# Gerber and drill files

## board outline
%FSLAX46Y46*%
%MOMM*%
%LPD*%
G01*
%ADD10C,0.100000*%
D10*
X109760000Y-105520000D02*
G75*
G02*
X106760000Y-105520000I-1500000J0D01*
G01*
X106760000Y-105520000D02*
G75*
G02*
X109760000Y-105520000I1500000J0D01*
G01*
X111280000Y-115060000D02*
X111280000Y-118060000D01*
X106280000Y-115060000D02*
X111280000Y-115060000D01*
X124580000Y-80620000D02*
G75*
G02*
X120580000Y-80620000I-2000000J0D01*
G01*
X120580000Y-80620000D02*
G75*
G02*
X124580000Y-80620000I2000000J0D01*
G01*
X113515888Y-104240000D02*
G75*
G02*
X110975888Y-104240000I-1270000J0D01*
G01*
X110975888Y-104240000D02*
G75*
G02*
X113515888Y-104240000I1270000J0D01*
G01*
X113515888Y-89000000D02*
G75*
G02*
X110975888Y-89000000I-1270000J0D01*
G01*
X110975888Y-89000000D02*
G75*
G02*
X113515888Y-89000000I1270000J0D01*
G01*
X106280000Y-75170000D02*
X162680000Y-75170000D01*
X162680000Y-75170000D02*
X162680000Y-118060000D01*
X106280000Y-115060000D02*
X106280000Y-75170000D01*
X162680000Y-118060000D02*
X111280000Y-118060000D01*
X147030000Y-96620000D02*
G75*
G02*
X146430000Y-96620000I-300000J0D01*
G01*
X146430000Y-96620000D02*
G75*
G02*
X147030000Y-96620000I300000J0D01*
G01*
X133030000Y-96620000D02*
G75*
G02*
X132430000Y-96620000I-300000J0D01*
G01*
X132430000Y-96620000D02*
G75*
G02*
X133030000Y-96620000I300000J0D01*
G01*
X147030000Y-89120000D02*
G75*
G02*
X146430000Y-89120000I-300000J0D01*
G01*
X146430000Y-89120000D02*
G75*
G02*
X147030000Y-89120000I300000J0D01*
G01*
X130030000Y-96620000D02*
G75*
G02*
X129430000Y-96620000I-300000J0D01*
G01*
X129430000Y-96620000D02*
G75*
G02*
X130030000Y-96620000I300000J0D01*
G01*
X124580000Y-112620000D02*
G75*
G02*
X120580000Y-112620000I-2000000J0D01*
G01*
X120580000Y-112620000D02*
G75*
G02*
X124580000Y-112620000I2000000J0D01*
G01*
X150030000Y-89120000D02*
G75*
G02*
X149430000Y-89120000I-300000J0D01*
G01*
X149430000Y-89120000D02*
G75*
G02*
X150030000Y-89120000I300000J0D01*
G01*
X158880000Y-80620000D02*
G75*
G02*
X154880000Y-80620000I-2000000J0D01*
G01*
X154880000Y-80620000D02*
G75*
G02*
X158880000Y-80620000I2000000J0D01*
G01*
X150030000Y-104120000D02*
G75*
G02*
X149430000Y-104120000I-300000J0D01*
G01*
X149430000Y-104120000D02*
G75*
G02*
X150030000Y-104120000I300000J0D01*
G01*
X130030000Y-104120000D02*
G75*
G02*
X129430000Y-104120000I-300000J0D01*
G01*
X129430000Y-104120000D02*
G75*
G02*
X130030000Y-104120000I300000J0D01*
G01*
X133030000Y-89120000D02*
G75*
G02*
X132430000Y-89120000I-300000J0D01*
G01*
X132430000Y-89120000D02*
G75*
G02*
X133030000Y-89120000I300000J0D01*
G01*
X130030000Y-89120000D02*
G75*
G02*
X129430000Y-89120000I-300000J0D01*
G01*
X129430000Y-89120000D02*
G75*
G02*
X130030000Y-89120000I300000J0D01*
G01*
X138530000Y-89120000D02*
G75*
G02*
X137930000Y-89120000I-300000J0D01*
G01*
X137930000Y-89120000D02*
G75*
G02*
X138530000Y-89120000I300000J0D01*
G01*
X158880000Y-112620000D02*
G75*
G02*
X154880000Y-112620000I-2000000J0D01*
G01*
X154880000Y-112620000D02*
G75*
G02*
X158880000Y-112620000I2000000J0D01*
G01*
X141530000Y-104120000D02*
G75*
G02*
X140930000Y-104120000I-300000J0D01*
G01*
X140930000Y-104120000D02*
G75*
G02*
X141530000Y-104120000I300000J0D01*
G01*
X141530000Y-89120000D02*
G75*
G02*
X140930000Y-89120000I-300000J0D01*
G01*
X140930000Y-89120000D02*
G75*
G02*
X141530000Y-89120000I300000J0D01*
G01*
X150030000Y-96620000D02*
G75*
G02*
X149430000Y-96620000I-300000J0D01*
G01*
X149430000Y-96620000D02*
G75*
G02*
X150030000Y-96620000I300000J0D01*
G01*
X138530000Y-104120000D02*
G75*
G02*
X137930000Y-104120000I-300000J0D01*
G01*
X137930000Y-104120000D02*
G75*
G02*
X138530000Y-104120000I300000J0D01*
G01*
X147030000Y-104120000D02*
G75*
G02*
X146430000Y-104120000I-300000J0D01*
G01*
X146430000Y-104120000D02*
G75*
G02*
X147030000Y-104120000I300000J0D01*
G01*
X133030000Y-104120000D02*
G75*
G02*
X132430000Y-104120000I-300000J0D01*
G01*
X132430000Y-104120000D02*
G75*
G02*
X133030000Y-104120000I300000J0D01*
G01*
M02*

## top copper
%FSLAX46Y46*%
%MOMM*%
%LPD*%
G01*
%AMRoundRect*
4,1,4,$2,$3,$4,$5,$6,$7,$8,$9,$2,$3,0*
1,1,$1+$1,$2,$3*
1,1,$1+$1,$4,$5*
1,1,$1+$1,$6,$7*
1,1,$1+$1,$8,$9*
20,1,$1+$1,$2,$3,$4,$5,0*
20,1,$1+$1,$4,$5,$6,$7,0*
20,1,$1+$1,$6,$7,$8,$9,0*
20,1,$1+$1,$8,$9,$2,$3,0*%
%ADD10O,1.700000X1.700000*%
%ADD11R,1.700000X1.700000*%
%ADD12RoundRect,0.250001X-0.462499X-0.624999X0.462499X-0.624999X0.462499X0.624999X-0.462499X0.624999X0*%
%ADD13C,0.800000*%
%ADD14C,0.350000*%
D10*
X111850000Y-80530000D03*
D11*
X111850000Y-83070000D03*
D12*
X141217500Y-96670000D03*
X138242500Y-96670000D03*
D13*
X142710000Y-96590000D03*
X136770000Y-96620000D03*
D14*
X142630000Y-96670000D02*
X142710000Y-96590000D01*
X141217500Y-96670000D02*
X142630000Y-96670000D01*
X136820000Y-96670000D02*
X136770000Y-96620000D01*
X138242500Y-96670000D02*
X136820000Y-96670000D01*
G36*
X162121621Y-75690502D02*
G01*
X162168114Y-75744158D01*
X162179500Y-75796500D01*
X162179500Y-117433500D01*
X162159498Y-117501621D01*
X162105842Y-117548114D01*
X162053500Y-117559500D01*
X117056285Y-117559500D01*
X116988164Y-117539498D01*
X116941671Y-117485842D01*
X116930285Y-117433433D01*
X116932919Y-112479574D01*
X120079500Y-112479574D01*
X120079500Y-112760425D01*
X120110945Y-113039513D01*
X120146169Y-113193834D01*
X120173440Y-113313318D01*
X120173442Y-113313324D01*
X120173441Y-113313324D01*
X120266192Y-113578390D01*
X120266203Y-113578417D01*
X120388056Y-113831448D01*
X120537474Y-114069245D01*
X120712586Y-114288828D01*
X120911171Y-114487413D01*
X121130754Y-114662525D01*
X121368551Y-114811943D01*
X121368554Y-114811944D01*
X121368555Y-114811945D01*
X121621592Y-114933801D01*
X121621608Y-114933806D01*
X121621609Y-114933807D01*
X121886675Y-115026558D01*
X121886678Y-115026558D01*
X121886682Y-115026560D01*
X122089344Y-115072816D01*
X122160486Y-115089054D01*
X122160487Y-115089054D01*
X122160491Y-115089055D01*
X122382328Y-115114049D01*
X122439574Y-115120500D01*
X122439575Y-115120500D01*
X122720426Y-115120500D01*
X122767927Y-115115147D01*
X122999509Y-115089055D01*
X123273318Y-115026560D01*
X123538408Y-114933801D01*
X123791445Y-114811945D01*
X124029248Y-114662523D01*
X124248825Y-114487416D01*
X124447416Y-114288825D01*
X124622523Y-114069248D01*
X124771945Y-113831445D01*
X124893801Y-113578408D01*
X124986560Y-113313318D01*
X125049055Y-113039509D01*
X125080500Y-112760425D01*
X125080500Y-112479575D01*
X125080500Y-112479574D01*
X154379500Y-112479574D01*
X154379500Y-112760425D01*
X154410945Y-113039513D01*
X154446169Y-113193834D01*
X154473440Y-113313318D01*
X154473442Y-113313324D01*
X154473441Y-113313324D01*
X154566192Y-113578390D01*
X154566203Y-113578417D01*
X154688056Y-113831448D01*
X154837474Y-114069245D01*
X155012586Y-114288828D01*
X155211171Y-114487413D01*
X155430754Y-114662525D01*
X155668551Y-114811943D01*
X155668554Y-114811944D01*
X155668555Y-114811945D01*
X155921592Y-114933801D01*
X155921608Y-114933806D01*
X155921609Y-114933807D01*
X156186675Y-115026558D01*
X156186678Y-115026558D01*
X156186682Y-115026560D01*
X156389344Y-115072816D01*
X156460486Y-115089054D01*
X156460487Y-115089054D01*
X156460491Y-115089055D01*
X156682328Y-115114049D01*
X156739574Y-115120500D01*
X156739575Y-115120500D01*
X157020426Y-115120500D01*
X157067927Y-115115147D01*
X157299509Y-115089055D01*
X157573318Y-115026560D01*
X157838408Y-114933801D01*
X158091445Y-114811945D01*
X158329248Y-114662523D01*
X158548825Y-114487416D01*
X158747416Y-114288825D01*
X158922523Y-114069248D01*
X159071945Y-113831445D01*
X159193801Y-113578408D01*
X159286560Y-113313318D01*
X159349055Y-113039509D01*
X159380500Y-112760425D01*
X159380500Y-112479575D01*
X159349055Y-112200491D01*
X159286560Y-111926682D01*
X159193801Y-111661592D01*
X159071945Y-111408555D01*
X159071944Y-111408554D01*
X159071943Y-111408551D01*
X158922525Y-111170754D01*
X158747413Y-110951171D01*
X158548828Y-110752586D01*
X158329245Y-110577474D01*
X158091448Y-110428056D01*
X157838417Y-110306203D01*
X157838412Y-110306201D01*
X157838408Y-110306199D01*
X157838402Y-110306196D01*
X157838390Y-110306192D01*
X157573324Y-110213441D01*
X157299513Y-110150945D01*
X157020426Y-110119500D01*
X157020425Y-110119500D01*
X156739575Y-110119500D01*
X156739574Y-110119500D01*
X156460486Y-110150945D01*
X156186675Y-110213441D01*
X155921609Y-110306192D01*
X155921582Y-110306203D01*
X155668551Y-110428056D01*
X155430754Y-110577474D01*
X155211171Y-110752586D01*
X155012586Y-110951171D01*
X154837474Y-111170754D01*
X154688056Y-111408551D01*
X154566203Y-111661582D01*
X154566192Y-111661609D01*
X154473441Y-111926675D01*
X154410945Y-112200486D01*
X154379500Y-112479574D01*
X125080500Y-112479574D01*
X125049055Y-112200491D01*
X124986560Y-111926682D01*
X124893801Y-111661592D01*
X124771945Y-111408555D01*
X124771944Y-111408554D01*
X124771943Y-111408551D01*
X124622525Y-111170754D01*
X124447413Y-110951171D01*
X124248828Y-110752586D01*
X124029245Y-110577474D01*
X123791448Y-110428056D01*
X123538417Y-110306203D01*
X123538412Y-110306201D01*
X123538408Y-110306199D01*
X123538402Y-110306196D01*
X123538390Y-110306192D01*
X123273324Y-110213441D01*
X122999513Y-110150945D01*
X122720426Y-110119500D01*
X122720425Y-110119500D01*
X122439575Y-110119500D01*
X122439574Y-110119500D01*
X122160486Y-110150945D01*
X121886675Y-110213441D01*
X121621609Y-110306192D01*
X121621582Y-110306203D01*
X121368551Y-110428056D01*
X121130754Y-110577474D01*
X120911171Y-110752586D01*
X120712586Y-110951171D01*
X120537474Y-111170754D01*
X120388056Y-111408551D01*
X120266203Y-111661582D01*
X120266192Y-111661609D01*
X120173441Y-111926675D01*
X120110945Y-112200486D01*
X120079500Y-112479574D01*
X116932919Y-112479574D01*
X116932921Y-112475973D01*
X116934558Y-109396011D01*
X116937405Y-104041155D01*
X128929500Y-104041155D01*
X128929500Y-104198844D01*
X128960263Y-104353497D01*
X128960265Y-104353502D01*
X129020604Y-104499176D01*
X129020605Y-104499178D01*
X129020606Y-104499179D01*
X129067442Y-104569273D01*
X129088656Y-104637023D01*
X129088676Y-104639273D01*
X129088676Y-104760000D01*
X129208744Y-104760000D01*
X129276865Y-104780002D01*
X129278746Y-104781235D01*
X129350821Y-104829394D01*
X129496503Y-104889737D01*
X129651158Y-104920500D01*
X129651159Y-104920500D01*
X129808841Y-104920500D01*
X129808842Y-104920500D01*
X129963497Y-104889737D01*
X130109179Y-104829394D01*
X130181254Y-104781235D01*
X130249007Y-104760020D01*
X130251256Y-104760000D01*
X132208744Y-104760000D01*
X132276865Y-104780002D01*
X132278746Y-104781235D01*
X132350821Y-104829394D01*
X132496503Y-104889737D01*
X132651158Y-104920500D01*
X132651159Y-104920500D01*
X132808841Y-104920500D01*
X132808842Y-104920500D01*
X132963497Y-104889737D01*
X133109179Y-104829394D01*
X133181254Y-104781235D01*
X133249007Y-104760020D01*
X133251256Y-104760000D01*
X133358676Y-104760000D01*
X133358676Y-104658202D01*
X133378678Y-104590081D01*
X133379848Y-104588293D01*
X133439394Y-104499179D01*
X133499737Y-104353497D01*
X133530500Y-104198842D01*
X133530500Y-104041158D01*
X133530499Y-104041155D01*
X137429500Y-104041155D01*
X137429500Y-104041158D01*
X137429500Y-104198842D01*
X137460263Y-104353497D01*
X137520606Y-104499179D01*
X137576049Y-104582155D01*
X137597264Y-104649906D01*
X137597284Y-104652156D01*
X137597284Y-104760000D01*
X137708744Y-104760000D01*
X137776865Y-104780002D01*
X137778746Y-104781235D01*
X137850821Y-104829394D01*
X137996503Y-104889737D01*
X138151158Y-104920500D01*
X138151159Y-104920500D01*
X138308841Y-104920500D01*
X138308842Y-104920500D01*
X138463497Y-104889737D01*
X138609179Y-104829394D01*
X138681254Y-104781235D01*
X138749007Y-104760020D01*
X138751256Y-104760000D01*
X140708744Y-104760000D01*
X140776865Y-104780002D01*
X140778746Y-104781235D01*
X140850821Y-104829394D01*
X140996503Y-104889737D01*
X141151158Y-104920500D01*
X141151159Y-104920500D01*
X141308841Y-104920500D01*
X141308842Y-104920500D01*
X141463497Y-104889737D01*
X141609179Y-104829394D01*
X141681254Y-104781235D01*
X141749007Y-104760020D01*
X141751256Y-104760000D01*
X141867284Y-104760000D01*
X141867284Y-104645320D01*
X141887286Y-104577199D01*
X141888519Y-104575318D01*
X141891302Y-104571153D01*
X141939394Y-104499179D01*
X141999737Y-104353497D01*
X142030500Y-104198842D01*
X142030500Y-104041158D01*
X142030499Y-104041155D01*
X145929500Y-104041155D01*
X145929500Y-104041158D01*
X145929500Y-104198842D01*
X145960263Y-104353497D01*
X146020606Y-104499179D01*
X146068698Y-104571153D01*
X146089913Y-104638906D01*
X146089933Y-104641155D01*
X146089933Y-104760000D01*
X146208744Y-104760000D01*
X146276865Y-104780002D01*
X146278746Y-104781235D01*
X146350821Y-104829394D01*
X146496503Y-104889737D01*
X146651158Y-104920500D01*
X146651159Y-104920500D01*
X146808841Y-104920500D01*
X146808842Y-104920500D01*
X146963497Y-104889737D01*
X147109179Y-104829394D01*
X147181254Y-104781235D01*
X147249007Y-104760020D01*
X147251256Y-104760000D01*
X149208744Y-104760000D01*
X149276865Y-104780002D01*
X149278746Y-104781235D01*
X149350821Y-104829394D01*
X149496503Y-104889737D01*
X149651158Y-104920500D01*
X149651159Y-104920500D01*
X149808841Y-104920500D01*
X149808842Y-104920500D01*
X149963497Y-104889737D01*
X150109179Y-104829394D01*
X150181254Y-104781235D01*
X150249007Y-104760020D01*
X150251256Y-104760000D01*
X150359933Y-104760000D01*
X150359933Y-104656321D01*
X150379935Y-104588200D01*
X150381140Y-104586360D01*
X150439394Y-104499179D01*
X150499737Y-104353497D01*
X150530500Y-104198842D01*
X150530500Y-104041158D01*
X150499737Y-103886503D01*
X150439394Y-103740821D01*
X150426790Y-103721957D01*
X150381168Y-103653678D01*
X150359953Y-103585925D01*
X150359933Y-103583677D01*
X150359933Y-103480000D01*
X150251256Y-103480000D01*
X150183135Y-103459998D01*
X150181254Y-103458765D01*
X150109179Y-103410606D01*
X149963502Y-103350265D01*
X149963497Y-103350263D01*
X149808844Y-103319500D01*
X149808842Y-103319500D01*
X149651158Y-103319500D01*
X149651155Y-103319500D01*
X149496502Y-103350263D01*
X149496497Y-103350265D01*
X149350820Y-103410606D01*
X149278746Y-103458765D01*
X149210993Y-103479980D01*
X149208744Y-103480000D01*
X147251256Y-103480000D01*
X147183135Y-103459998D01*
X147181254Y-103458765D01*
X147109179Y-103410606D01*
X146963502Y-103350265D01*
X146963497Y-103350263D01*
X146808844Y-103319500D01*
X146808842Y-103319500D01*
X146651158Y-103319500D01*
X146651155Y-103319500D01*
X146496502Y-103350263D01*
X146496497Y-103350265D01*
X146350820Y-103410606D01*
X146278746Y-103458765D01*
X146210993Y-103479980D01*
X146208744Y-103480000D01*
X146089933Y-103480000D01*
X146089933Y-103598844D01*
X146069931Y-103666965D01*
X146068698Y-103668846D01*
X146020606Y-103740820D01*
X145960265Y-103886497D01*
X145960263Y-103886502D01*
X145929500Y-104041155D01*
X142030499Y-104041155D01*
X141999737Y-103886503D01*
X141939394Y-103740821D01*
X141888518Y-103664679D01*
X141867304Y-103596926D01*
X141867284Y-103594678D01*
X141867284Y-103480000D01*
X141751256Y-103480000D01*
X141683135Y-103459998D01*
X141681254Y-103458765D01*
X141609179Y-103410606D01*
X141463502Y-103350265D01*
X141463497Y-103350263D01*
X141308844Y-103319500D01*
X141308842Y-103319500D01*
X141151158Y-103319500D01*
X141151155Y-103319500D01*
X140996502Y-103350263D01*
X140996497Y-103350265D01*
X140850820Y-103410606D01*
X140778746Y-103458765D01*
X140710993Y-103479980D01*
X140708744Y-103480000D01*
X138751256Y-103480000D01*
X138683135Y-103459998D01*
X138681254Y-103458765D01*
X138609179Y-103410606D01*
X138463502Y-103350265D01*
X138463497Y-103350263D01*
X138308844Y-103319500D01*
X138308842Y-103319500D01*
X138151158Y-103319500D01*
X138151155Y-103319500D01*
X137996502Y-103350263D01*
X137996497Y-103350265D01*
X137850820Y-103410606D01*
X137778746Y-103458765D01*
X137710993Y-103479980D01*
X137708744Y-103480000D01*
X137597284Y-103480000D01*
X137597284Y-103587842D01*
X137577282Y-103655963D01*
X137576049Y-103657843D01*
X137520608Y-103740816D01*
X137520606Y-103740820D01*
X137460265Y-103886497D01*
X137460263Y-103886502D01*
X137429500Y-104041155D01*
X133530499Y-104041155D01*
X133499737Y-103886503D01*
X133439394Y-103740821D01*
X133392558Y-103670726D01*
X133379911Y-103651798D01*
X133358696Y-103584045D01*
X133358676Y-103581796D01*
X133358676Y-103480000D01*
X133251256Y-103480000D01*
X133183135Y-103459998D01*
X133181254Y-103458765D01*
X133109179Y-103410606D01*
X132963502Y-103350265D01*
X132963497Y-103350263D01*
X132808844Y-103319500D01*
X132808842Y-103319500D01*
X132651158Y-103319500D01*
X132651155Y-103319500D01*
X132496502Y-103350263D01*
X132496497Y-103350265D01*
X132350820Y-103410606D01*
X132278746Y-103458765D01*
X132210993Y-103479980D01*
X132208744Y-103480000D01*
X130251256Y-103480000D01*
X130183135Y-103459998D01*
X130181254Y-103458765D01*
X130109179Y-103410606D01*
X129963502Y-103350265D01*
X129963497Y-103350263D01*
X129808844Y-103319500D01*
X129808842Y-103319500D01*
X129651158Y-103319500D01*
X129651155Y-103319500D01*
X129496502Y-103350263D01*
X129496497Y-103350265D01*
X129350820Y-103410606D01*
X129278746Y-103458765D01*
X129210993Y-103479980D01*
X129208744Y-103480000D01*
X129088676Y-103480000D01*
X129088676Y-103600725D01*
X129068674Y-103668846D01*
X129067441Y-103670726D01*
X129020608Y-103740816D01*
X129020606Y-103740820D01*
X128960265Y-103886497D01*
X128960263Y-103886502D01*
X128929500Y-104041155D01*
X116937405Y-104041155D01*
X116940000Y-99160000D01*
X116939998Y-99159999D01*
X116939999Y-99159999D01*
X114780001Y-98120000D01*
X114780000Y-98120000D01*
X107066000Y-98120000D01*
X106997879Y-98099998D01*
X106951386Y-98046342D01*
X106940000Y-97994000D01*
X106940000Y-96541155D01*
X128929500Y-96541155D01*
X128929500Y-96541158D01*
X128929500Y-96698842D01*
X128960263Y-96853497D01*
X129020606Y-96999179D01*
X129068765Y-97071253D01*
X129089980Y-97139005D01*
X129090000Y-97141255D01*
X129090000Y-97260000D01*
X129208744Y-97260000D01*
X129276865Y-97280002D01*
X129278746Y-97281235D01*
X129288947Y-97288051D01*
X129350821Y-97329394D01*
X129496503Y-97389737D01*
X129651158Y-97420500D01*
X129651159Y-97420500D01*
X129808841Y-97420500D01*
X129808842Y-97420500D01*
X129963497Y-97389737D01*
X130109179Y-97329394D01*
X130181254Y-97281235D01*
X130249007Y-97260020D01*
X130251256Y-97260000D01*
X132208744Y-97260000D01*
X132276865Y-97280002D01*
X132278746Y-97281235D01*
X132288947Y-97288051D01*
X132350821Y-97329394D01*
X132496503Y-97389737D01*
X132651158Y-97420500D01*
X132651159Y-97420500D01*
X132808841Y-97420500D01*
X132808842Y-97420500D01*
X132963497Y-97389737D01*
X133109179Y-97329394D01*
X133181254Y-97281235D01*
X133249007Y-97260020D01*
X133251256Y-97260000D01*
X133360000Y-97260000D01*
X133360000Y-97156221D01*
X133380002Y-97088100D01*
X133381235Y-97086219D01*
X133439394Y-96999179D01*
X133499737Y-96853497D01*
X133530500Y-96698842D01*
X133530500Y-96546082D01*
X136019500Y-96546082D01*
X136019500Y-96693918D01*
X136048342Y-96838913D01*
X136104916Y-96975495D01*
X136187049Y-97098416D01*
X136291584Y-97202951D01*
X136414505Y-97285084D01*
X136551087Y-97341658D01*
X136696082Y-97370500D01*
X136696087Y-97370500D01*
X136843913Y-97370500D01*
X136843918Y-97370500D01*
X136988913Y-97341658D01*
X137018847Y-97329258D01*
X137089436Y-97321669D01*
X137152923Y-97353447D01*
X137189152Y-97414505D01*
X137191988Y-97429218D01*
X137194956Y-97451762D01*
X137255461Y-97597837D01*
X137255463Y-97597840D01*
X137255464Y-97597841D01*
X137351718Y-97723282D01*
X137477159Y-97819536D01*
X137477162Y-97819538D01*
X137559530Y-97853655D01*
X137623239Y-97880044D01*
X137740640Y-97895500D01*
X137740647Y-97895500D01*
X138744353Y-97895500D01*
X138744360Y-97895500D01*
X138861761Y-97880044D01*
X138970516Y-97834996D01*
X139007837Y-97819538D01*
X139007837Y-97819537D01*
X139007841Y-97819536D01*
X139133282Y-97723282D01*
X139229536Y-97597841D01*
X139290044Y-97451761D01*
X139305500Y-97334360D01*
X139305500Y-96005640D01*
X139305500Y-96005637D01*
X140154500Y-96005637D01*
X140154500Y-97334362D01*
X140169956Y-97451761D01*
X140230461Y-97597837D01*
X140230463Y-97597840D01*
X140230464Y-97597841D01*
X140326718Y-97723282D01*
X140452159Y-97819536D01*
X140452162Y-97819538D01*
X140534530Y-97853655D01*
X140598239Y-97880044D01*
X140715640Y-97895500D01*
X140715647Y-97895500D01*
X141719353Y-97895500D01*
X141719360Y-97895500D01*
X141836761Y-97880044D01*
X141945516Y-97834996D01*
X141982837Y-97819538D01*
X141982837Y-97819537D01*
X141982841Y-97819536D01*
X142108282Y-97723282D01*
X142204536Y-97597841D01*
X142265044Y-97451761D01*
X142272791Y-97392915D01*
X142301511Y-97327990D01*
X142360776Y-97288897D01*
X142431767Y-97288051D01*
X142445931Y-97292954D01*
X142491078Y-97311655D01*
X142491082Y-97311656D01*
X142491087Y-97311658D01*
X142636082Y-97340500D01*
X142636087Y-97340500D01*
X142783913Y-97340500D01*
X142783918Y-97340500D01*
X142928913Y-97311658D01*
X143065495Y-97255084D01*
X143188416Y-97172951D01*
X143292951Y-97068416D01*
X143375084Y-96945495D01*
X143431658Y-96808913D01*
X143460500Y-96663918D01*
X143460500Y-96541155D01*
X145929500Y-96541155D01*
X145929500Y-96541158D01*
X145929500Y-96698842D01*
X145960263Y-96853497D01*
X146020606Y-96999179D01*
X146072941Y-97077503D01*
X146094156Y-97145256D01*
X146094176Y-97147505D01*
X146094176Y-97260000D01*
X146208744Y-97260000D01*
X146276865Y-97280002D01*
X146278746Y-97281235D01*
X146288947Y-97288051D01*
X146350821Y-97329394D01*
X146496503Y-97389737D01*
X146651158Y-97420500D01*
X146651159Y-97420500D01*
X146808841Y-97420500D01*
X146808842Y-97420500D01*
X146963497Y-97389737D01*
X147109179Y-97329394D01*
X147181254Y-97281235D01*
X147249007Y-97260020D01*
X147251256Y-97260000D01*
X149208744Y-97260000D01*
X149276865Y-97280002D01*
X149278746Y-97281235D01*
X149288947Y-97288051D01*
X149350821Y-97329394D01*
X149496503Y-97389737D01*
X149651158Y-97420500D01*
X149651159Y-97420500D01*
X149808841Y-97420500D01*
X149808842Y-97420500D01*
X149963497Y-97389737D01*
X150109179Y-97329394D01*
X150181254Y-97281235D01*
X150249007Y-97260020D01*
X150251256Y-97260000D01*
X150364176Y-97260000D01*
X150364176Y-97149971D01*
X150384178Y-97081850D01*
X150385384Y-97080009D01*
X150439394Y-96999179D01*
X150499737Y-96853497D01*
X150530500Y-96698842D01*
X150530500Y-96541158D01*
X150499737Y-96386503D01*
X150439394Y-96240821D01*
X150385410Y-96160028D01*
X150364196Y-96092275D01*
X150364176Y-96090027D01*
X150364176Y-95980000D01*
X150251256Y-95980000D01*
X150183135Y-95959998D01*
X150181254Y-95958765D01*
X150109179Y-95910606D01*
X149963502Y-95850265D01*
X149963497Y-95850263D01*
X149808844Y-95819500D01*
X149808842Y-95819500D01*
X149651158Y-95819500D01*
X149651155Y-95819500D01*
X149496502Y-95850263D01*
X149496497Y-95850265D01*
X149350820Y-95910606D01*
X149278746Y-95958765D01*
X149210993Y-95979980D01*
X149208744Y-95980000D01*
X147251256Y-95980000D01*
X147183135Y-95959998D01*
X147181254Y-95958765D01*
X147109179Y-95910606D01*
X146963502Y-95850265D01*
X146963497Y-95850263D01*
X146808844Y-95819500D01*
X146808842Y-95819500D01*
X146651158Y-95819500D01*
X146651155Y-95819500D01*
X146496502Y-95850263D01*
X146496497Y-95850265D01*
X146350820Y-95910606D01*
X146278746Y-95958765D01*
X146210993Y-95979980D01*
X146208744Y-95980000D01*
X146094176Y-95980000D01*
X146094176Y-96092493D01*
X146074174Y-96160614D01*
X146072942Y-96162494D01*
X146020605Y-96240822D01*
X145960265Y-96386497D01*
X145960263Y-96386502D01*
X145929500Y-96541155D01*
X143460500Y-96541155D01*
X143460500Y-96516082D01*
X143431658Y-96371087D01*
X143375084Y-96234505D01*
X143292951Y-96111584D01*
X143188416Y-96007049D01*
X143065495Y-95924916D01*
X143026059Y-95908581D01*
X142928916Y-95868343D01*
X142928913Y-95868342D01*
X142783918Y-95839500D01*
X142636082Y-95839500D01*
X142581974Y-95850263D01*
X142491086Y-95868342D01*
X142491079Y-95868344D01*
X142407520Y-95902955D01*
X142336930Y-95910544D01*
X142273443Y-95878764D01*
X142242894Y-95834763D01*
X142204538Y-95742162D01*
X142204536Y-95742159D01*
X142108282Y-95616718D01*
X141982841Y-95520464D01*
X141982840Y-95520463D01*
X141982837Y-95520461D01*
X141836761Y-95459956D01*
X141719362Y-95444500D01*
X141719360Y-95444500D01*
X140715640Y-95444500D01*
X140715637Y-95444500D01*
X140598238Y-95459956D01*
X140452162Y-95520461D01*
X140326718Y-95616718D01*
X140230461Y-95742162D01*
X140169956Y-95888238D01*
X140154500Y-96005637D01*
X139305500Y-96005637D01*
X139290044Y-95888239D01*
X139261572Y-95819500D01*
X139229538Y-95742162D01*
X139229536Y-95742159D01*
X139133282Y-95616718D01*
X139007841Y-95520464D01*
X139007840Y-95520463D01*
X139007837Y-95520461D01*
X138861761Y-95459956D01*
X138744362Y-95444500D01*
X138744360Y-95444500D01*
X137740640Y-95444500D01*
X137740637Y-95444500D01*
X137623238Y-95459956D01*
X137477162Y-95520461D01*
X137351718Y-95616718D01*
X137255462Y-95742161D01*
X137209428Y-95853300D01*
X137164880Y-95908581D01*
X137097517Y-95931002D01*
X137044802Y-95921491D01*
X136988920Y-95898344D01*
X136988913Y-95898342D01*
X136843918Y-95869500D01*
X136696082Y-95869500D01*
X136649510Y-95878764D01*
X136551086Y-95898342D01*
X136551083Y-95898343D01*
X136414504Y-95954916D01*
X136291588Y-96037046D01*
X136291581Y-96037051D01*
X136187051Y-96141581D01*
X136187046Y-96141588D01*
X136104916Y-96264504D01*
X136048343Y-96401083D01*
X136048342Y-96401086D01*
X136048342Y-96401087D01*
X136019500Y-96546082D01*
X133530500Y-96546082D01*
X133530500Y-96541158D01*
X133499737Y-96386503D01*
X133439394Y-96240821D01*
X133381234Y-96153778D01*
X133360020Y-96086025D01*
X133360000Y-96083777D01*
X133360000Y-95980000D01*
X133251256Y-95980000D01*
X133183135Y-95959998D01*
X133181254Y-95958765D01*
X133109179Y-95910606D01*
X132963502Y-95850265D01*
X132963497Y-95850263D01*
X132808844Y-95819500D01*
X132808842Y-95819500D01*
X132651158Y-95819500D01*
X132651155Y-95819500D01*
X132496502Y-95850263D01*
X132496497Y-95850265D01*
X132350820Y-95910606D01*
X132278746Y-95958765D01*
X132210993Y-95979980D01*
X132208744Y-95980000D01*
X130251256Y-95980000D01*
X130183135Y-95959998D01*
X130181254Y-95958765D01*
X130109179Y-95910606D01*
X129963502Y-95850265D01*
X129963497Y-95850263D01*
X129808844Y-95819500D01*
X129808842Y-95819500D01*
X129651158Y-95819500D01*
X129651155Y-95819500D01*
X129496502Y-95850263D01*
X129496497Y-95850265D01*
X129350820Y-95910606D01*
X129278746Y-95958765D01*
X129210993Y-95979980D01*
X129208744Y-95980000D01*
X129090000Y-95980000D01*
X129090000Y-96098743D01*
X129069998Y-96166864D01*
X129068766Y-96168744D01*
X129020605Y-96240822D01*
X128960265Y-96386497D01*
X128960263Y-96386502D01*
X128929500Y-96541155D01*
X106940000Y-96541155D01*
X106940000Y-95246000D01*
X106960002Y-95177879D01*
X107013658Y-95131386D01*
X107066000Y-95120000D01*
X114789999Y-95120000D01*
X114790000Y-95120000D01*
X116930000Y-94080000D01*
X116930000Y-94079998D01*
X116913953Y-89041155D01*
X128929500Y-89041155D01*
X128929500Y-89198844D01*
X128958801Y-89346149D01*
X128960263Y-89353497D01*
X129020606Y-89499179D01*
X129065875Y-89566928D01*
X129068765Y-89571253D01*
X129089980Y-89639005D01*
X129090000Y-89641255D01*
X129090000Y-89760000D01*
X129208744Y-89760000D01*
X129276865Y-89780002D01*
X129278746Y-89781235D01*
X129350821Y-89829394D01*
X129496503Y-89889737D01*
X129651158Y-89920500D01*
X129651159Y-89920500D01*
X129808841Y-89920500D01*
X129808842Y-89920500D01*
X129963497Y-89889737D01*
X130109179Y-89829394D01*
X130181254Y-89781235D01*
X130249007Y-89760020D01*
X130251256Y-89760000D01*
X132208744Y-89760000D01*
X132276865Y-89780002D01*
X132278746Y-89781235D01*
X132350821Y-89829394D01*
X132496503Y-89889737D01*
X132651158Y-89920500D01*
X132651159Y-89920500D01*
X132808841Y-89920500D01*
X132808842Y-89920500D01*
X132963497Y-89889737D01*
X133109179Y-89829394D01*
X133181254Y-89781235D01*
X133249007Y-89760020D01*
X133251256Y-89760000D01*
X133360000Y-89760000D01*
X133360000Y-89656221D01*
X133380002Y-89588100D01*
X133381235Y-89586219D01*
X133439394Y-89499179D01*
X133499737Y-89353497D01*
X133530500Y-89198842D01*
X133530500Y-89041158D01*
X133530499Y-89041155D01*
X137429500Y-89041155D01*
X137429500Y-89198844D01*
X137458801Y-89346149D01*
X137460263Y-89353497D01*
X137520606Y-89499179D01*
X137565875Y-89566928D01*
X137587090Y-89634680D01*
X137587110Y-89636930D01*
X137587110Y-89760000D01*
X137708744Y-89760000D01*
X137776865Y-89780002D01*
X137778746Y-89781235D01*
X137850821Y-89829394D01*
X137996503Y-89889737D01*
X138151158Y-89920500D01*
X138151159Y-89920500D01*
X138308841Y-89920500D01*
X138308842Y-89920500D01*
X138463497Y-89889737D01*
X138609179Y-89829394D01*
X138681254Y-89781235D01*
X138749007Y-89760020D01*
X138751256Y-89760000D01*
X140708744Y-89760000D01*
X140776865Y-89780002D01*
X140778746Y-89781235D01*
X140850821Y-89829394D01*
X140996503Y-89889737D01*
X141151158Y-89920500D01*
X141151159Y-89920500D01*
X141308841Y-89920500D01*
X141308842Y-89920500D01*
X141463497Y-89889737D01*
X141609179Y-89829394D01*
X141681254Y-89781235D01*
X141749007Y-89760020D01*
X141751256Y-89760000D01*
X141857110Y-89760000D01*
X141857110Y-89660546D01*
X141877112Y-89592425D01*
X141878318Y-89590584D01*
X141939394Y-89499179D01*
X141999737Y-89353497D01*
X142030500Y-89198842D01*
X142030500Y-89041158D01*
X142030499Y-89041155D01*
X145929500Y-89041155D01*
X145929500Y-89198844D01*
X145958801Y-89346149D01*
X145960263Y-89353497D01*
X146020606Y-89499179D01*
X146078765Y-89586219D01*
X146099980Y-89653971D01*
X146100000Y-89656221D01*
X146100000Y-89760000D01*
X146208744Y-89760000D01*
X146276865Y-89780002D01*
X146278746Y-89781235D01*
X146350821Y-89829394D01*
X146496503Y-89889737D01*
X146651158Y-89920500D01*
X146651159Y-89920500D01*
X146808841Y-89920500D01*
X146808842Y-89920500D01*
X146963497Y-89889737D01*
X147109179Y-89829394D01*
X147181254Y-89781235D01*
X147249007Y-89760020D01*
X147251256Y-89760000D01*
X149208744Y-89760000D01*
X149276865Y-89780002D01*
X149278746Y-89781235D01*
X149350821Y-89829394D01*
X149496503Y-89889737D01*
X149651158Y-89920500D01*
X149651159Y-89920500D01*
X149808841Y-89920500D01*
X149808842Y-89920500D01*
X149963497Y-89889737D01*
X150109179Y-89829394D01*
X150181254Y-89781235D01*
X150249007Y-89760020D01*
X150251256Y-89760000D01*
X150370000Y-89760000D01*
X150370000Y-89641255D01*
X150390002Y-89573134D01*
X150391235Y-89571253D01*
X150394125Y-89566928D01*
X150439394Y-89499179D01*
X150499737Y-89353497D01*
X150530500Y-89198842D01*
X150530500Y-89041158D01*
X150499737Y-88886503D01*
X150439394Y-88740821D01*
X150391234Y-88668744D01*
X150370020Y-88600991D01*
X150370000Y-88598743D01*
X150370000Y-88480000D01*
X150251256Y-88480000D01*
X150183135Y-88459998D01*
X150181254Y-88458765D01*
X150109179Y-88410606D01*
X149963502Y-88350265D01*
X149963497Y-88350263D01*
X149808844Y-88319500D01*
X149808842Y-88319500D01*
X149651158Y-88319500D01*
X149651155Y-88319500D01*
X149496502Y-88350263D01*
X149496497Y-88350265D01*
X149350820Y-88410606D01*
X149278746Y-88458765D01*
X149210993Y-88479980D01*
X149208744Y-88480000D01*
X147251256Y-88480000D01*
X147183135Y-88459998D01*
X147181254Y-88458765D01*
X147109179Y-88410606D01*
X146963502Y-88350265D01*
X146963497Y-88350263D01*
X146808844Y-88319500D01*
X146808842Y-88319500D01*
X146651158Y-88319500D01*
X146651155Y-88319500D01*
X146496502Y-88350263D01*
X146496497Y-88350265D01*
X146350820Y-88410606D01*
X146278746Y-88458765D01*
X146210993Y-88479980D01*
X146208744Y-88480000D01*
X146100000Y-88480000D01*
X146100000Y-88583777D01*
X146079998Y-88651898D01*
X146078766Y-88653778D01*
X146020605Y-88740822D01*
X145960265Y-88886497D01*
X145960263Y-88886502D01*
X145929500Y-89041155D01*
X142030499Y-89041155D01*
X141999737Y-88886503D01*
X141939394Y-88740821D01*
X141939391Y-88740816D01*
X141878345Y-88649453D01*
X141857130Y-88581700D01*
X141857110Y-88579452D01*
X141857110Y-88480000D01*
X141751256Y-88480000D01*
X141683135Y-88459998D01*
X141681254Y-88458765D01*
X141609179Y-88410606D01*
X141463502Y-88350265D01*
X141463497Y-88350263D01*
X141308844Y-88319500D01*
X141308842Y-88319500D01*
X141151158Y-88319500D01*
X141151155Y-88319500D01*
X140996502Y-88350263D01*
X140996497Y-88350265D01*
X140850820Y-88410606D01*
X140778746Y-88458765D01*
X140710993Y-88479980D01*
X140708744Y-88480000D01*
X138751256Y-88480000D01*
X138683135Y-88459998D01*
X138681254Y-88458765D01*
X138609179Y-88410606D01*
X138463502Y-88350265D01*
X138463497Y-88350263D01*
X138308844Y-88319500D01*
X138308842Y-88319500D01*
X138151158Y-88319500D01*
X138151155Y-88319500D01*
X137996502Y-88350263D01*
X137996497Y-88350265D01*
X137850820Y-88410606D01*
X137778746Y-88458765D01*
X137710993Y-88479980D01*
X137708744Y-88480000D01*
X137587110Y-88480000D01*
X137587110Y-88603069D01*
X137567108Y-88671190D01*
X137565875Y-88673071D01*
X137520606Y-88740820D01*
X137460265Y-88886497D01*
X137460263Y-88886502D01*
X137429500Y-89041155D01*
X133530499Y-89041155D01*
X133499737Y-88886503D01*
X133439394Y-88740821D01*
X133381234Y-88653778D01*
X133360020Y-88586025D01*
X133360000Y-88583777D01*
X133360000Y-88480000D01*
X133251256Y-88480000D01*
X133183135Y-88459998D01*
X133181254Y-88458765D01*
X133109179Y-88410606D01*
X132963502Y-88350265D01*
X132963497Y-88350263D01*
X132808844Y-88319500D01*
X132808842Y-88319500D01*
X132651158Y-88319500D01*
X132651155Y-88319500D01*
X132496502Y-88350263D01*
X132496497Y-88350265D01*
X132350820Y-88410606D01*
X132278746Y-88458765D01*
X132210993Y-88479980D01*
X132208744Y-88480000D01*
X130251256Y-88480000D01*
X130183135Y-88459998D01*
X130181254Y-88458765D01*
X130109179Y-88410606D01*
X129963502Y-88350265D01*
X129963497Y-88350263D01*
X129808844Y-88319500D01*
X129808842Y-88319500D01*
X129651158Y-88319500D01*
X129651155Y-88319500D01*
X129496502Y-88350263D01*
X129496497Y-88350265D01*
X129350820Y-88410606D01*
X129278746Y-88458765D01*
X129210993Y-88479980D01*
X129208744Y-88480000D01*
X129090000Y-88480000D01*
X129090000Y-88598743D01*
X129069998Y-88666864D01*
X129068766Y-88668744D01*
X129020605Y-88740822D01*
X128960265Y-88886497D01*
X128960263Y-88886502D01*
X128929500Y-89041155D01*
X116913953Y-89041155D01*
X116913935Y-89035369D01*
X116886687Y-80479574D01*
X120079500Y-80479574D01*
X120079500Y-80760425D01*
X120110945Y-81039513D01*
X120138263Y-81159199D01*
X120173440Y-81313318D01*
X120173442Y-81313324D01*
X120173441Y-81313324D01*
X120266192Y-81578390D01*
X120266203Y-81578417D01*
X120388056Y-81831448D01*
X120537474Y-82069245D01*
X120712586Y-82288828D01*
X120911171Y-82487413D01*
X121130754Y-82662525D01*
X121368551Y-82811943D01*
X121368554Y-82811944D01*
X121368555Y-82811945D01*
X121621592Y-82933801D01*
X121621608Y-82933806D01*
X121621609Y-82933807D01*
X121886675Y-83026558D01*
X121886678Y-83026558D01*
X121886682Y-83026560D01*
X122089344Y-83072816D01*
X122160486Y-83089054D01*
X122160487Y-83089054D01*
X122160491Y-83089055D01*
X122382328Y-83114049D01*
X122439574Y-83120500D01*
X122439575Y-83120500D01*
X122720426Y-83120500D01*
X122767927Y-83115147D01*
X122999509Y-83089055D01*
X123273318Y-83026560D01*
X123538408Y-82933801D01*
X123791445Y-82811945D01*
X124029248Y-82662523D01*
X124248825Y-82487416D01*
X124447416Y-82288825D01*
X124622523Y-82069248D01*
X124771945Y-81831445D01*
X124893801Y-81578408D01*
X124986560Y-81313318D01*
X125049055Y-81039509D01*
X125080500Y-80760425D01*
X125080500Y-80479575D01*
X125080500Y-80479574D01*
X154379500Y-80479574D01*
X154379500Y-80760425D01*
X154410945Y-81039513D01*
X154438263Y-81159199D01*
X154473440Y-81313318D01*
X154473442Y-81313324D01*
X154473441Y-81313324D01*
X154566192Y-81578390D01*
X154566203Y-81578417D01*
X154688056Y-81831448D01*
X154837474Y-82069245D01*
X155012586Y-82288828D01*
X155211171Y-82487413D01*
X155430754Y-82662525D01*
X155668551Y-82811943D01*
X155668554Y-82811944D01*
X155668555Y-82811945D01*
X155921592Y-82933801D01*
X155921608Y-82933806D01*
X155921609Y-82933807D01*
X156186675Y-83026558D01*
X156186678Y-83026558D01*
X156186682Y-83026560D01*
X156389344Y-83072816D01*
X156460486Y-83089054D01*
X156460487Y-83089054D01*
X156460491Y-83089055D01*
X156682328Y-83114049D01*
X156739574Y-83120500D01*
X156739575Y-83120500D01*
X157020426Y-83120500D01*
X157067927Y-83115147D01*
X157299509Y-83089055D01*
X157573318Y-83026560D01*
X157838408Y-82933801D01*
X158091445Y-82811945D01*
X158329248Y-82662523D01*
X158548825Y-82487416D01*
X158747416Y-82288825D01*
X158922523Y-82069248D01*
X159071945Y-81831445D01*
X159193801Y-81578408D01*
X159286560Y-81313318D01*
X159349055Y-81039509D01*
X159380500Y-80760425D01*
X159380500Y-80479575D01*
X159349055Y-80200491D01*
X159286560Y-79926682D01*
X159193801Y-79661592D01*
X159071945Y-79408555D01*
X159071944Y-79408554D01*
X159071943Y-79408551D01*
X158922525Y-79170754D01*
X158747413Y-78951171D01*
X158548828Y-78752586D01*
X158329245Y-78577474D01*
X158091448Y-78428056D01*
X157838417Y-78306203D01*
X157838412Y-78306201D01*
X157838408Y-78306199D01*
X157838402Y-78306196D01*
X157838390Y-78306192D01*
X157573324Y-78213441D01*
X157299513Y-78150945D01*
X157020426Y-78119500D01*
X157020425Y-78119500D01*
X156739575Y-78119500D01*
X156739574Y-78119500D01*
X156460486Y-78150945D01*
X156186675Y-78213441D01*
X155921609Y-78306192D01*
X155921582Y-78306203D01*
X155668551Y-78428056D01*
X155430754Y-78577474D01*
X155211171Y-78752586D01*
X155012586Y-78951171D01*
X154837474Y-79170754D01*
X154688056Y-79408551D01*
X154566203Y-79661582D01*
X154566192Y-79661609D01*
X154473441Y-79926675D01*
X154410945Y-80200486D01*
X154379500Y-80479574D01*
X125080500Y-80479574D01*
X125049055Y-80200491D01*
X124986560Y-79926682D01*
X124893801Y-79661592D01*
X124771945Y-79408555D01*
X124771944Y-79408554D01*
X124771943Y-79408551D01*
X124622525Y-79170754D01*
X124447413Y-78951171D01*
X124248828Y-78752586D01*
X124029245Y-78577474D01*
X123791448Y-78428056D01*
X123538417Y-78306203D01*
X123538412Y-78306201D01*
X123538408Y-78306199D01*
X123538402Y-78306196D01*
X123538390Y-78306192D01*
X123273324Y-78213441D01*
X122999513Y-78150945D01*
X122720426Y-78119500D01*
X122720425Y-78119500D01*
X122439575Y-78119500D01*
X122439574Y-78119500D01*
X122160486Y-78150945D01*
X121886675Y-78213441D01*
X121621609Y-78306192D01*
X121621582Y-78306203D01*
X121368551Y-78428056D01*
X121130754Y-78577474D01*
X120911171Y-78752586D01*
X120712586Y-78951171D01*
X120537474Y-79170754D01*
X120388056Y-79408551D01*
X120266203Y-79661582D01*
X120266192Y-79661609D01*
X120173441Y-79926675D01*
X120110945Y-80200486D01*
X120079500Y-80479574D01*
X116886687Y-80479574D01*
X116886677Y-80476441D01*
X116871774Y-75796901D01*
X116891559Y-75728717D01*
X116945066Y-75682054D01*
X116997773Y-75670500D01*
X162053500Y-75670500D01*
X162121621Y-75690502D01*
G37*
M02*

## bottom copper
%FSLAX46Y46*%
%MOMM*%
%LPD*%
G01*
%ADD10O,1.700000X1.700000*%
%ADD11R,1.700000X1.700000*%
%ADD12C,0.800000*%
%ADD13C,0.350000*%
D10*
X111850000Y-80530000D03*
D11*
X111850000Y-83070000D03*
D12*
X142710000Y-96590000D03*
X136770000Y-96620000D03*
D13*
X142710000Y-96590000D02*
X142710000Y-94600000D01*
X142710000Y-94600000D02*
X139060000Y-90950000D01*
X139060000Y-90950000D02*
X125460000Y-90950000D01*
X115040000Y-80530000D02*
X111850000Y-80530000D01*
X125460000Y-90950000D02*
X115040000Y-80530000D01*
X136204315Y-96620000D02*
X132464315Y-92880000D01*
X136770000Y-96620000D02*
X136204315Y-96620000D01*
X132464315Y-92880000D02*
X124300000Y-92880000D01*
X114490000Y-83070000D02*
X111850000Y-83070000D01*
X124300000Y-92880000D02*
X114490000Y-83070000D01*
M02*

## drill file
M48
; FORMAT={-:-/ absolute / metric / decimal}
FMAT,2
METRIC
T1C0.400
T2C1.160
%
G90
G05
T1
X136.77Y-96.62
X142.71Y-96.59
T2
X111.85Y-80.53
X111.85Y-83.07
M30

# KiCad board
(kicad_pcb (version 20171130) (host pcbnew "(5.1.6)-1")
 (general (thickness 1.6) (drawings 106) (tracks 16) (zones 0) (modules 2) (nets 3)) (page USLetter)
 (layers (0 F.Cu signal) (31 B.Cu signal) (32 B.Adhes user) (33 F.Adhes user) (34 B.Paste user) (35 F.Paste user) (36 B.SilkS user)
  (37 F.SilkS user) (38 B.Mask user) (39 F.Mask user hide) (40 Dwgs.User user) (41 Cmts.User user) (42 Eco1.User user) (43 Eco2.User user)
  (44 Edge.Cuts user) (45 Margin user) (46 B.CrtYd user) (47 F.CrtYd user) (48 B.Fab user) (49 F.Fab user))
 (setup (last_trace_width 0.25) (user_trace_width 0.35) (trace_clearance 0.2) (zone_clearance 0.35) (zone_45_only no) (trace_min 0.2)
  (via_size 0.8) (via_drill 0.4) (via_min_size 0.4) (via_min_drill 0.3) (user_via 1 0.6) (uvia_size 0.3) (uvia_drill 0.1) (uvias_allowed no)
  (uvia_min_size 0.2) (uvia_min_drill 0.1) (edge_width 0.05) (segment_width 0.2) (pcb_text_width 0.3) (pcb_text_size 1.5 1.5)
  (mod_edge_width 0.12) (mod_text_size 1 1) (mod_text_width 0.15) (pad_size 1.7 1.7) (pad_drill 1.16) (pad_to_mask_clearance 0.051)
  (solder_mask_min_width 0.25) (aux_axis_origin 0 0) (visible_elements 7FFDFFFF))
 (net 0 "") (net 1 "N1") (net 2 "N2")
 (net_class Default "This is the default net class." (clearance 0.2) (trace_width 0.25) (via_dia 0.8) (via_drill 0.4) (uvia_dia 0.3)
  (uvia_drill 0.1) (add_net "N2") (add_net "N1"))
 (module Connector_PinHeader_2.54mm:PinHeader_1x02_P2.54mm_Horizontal (layer F.Cu) (at 111.85 83.07 180)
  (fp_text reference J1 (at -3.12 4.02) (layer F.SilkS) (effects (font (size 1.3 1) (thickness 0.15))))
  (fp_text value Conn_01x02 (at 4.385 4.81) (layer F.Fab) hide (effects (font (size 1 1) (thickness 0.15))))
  (pad 2 thru_hole oval (at 0 2.54 180) (size 1.7 1.7) (drill 1.16) (layers *.Cu *.Mask) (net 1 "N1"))
  (pad 1 thru_hole rect (at 0 0 180) (size 1.7 1.7) (drill 1.16) (layers *.Cu *.Mask) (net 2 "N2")))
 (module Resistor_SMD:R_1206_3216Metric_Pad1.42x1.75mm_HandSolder (layer F.Cu) (at 139.73 96.67)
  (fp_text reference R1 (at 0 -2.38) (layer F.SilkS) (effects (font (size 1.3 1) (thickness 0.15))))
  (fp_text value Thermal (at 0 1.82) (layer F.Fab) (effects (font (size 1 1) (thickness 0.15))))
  (pad 2 smd roundrect (at 1.4875 0) (size 1.425 1.75) (layers F.Cu F.Paste F.Mask) (roundrect_rratio 0.175439) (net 1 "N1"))
  (pad 1 smd roundrect (at -1.4875 0) (size 1.425 1.75) (layers F.Cu F.Paste F.Mask) (roundrect_rratio 0.175439) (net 2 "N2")))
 (gr_circle (center 108.26 105.52) (end 109.76 105.52) (layer Edge.Cuts) (width 0.1))
 (gr_line (start 111.28 115.06) (end 111.28 118.06) (layer Edge.Cuts) (width 0.1))
 (gr_line (start 106.28 115.06) (end 111.28 115.06) (layer Edge.Cuts) (width 0.1))
 (gr_circle (center 122.58 80.62) (end 124.58 80.62) (layer Edge.Cuts) (width 0.1))
 (gr_circle (center 112.245888 104.24) (end 113.515888 104.24) (layer Edge.Cuts) (width 0.1))
 (gr_circle (center 112.245888 89) (end 113.515888 89) (layer Edge.Cuts) (width 0.1))
 (gr_line (start 106.28 75.17) (end 162.68 75.17) (layer Edge.Cuts) (width 0.1))
 (gr_line (start 162.68 75.17) (end 162.68 118.06) (layer Edge.Cuts) (width 0.1))
 (gr_line (start 106.28 115.06) (end 106.28 75.17) (layer Edge.Cuts) (width 0.1))
 (gr_line (start 162.68 118.06) (end 111.28 118.06) (layer Edge.Cuts) (width 0.1))
 (gr_circle (center 146.73 96.62) (end 147.03 96.62) (layer Edge.Cuts) (width 0.1))
 (gr_circle (center 132.73 96.62) (end 133.03 96.62) (layer Edge.Cuts) (width 0.1))
 (gr_circle (center 146.73 89.12) (end 147.03 89.12) (layer Edge.Cuts) (width 0.1))
 (gr_circle (center 129.73 96.62) (end 130.03 96.62) (layer Edge.Cuts) (width 0.1))
 (gr_circle (center 122.58 112.62) (end 124.58 112.62) (layer Edge.Cuts) (width 0.1))
 (gr_circle (center 149.73 89.12) (end 150.03 89.12) (layer Edge.Cuts) (width 0.1))
 (gr_circle (center 156.88 80.62) (end 158.88 80.62) (layer Edge.Cuts) (width 0.1))
 (gr_circle (center 149.73 104.12) (end 150.03 104.12) (layer Edge.Cuts) (width 0.1))
 (gr_circle (center 129.73 104.12) (end 130.03 104.12) (layer Edge.Cuts) (width 0.1))
 (gr_circle (center 132.73 89.12) (end 133.03 89.12) (layer Edge.Cuts) (width 0.1))
 (gr_circle (center 129.73 89.12) (end 130.03 89.12) (layer Edge.Cuts) (width 0.1))
 (gr_circle (center 138.23 89.12) (end 138.53 89.12) (layer Edge.Cuts) (width 0.1))
 (gr_circle (center 156.88 112.62) (end 158.88 112.62) (layer Edge.Cuts) (width 0.1))
 (gr_circle (center 141.23 104.12) (end 141.53 104.12) (layer Edge.Cuts) (width 0.1))
 (gr_circle (center 141.23 89.12) (end 141.53 89.12) (layer Edge.Cuts) (width 0.1))
 (gr_circle (center 149.73 96.62) (end 150.03 96.62) (layer Edge.Cuts) (width 0.1))
 (gr_circle (center 138.23 104.12) (end 138.53 104.12) (layer Edge.Cuts) (width 0.1))
 (gr_circle (center 146.73 104.12) (end 147.03 104.12) (layer Edge.Cuts) (width 0.1))
 (gr_circle (center 132.73 104.12) (end 133.03 104.12) (layer Edge.Cuts) (width 0.1))
 (via (at 142.71 96.59) (size 0.8) (drill 0.4) (layers F.Cu B.Cu) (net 1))
 (segment (start 142.63 96.67) (end 142.71 96.59) (width 0.35) (layer F.Cu) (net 1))
 (segment (start 141.2175 96.67) (end 142.63 96.67) (width 0.35) (layer F.Cu) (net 1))
 (segment (start 142.71 96.59) (end 142.71 94.6) (width 0.35) (layer B.Cu) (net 1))
 (segment (start 142.71 94.6) (end 139.06 90.95) (width 0.35) (layer B.Cu) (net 1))
 (segment (start 139.06 90.95) (end 125.46 90.95) (width 0.35) (layer B.Cu) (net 1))
 (segment (start 115.04 80.53) (end 111.85 80.53) (width 0.35) (layer B.Cu) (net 1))
 (segment (start 125.46 90.95) (end 115.04 80.53) (width 0.35) (layer B.Cu) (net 1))
 (via (at 136.77 96.62) (size 0.8) (drill 0.4) (layers F.Cu B.Cu) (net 2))
 (segment (start 136.82 96.67) (end 136.77 96.62) (width 0.35) (layer F.Cu) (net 2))
 (segment (start 138.2425 96.67) (end 136.82 96.67) (width 0.35) (layer F.Cu) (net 2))
 (segment (start 136.204315 96.62) (end 132.464315 92.88) (width 0.35) (layer B.Cu) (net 2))
 (segment (start 136.77 96.62) (end 136.204315 96.62) (width 0.35) (layer B.Cu) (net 2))
 (segment (start 132.464315 92.88) (end 124.3 92.88) (width 0.35) (layer B.Cu) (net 2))
 (segment (start 114.49 83.07) (end 111.85 83.07) (width 0.35) (layer B.Cu) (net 2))
 (segment (start 124.3 92.88) (end 114.49 83.07) (width 0.35) (layer B.Cu) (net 2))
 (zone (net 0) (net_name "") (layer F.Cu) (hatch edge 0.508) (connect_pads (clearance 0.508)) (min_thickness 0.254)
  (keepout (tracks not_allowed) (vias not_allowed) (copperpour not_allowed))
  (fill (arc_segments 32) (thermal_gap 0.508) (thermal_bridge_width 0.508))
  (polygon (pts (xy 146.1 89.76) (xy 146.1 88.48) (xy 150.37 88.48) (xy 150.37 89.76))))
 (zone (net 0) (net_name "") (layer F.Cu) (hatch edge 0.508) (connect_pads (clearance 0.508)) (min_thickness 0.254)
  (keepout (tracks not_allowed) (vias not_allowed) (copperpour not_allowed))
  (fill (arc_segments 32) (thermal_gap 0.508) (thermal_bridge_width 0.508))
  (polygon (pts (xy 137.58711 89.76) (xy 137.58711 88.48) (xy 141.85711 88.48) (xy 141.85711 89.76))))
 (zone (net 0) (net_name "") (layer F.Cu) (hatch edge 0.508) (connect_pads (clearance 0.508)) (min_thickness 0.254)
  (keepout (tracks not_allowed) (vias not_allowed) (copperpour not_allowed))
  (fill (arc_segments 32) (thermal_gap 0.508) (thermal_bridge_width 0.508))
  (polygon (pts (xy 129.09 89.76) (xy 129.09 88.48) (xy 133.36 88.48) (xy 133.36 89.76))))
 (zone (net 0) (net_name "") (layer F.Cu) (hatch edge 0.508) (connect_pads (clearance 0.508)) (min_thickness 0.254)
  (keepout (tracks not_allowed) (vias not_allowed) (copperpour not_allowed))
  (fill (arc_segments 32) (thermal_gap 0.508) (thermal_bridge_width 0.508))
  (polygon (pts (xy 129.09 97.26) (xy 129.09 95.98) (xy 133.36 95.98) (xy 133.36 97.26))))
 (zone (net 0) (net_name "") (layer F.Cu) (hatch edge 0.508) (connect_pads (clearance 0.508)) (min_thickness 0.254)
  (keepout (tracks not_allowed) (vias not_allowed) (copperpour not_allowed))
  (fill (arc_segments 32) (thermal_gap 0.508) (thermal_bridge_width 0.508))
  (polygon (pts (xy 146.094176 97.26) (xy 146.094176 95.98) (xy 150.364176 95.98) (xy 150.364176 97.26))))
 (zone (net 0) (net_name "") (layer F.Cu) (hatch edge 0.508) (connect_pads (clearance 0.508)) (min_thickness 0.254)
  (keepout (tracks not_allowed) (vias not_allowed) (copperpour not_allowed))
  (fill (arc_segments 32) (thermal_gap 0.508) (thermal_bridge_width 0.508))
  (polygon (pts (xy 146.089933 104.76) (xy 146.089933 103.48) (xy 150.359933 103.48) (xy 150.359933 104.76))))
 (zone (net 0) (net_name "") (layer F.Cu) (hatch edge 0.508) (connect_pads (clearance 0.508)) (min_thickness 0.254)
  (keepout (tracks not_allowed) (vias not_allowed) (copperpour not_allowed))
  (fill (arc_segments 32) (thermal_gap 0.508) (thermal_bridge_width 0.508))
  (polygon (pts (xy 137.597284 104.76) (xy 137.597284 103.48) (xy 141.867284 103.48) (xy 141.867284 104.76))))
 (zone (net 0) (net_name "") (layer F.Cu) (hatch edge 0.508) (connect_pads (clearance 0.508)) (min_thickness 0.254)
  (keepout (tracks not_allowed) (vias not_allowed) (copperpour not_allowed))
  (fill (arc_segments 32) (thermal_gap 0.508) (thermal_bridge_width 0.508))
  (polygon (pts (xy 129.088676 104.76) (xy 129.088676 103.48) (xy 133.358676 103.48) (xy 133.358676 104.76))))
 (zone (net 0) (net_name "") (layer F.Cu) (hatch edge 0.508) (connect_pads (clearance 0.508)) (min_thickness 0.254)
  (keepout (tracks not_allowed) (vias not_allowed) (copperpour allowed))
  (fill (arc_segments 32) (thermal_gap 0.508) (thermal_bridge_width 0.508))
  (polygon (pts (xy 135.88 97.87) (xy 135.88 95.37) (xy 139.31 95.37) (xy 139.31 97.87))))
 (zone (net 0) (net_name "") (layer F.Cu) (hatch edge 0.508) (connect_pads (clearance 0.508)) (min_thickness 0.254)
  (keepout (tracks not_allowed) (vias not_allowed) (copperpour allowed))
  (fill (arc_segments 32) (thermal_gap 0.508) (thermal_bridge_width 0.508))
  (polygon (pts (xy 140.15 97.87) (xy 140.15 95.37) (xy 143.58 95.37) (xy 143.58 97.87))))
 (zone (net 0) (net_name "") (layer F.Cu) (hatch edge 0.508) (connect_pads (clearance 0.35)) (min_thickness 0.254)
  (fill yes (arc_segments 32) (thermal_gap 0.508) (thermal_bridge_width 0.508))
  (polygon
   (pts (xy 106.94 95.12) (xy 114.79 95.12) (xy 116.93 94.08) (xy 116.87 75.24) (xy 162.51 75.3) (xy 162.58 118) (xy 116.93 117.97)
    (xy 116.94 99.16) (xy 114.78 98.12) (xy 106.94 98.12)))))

